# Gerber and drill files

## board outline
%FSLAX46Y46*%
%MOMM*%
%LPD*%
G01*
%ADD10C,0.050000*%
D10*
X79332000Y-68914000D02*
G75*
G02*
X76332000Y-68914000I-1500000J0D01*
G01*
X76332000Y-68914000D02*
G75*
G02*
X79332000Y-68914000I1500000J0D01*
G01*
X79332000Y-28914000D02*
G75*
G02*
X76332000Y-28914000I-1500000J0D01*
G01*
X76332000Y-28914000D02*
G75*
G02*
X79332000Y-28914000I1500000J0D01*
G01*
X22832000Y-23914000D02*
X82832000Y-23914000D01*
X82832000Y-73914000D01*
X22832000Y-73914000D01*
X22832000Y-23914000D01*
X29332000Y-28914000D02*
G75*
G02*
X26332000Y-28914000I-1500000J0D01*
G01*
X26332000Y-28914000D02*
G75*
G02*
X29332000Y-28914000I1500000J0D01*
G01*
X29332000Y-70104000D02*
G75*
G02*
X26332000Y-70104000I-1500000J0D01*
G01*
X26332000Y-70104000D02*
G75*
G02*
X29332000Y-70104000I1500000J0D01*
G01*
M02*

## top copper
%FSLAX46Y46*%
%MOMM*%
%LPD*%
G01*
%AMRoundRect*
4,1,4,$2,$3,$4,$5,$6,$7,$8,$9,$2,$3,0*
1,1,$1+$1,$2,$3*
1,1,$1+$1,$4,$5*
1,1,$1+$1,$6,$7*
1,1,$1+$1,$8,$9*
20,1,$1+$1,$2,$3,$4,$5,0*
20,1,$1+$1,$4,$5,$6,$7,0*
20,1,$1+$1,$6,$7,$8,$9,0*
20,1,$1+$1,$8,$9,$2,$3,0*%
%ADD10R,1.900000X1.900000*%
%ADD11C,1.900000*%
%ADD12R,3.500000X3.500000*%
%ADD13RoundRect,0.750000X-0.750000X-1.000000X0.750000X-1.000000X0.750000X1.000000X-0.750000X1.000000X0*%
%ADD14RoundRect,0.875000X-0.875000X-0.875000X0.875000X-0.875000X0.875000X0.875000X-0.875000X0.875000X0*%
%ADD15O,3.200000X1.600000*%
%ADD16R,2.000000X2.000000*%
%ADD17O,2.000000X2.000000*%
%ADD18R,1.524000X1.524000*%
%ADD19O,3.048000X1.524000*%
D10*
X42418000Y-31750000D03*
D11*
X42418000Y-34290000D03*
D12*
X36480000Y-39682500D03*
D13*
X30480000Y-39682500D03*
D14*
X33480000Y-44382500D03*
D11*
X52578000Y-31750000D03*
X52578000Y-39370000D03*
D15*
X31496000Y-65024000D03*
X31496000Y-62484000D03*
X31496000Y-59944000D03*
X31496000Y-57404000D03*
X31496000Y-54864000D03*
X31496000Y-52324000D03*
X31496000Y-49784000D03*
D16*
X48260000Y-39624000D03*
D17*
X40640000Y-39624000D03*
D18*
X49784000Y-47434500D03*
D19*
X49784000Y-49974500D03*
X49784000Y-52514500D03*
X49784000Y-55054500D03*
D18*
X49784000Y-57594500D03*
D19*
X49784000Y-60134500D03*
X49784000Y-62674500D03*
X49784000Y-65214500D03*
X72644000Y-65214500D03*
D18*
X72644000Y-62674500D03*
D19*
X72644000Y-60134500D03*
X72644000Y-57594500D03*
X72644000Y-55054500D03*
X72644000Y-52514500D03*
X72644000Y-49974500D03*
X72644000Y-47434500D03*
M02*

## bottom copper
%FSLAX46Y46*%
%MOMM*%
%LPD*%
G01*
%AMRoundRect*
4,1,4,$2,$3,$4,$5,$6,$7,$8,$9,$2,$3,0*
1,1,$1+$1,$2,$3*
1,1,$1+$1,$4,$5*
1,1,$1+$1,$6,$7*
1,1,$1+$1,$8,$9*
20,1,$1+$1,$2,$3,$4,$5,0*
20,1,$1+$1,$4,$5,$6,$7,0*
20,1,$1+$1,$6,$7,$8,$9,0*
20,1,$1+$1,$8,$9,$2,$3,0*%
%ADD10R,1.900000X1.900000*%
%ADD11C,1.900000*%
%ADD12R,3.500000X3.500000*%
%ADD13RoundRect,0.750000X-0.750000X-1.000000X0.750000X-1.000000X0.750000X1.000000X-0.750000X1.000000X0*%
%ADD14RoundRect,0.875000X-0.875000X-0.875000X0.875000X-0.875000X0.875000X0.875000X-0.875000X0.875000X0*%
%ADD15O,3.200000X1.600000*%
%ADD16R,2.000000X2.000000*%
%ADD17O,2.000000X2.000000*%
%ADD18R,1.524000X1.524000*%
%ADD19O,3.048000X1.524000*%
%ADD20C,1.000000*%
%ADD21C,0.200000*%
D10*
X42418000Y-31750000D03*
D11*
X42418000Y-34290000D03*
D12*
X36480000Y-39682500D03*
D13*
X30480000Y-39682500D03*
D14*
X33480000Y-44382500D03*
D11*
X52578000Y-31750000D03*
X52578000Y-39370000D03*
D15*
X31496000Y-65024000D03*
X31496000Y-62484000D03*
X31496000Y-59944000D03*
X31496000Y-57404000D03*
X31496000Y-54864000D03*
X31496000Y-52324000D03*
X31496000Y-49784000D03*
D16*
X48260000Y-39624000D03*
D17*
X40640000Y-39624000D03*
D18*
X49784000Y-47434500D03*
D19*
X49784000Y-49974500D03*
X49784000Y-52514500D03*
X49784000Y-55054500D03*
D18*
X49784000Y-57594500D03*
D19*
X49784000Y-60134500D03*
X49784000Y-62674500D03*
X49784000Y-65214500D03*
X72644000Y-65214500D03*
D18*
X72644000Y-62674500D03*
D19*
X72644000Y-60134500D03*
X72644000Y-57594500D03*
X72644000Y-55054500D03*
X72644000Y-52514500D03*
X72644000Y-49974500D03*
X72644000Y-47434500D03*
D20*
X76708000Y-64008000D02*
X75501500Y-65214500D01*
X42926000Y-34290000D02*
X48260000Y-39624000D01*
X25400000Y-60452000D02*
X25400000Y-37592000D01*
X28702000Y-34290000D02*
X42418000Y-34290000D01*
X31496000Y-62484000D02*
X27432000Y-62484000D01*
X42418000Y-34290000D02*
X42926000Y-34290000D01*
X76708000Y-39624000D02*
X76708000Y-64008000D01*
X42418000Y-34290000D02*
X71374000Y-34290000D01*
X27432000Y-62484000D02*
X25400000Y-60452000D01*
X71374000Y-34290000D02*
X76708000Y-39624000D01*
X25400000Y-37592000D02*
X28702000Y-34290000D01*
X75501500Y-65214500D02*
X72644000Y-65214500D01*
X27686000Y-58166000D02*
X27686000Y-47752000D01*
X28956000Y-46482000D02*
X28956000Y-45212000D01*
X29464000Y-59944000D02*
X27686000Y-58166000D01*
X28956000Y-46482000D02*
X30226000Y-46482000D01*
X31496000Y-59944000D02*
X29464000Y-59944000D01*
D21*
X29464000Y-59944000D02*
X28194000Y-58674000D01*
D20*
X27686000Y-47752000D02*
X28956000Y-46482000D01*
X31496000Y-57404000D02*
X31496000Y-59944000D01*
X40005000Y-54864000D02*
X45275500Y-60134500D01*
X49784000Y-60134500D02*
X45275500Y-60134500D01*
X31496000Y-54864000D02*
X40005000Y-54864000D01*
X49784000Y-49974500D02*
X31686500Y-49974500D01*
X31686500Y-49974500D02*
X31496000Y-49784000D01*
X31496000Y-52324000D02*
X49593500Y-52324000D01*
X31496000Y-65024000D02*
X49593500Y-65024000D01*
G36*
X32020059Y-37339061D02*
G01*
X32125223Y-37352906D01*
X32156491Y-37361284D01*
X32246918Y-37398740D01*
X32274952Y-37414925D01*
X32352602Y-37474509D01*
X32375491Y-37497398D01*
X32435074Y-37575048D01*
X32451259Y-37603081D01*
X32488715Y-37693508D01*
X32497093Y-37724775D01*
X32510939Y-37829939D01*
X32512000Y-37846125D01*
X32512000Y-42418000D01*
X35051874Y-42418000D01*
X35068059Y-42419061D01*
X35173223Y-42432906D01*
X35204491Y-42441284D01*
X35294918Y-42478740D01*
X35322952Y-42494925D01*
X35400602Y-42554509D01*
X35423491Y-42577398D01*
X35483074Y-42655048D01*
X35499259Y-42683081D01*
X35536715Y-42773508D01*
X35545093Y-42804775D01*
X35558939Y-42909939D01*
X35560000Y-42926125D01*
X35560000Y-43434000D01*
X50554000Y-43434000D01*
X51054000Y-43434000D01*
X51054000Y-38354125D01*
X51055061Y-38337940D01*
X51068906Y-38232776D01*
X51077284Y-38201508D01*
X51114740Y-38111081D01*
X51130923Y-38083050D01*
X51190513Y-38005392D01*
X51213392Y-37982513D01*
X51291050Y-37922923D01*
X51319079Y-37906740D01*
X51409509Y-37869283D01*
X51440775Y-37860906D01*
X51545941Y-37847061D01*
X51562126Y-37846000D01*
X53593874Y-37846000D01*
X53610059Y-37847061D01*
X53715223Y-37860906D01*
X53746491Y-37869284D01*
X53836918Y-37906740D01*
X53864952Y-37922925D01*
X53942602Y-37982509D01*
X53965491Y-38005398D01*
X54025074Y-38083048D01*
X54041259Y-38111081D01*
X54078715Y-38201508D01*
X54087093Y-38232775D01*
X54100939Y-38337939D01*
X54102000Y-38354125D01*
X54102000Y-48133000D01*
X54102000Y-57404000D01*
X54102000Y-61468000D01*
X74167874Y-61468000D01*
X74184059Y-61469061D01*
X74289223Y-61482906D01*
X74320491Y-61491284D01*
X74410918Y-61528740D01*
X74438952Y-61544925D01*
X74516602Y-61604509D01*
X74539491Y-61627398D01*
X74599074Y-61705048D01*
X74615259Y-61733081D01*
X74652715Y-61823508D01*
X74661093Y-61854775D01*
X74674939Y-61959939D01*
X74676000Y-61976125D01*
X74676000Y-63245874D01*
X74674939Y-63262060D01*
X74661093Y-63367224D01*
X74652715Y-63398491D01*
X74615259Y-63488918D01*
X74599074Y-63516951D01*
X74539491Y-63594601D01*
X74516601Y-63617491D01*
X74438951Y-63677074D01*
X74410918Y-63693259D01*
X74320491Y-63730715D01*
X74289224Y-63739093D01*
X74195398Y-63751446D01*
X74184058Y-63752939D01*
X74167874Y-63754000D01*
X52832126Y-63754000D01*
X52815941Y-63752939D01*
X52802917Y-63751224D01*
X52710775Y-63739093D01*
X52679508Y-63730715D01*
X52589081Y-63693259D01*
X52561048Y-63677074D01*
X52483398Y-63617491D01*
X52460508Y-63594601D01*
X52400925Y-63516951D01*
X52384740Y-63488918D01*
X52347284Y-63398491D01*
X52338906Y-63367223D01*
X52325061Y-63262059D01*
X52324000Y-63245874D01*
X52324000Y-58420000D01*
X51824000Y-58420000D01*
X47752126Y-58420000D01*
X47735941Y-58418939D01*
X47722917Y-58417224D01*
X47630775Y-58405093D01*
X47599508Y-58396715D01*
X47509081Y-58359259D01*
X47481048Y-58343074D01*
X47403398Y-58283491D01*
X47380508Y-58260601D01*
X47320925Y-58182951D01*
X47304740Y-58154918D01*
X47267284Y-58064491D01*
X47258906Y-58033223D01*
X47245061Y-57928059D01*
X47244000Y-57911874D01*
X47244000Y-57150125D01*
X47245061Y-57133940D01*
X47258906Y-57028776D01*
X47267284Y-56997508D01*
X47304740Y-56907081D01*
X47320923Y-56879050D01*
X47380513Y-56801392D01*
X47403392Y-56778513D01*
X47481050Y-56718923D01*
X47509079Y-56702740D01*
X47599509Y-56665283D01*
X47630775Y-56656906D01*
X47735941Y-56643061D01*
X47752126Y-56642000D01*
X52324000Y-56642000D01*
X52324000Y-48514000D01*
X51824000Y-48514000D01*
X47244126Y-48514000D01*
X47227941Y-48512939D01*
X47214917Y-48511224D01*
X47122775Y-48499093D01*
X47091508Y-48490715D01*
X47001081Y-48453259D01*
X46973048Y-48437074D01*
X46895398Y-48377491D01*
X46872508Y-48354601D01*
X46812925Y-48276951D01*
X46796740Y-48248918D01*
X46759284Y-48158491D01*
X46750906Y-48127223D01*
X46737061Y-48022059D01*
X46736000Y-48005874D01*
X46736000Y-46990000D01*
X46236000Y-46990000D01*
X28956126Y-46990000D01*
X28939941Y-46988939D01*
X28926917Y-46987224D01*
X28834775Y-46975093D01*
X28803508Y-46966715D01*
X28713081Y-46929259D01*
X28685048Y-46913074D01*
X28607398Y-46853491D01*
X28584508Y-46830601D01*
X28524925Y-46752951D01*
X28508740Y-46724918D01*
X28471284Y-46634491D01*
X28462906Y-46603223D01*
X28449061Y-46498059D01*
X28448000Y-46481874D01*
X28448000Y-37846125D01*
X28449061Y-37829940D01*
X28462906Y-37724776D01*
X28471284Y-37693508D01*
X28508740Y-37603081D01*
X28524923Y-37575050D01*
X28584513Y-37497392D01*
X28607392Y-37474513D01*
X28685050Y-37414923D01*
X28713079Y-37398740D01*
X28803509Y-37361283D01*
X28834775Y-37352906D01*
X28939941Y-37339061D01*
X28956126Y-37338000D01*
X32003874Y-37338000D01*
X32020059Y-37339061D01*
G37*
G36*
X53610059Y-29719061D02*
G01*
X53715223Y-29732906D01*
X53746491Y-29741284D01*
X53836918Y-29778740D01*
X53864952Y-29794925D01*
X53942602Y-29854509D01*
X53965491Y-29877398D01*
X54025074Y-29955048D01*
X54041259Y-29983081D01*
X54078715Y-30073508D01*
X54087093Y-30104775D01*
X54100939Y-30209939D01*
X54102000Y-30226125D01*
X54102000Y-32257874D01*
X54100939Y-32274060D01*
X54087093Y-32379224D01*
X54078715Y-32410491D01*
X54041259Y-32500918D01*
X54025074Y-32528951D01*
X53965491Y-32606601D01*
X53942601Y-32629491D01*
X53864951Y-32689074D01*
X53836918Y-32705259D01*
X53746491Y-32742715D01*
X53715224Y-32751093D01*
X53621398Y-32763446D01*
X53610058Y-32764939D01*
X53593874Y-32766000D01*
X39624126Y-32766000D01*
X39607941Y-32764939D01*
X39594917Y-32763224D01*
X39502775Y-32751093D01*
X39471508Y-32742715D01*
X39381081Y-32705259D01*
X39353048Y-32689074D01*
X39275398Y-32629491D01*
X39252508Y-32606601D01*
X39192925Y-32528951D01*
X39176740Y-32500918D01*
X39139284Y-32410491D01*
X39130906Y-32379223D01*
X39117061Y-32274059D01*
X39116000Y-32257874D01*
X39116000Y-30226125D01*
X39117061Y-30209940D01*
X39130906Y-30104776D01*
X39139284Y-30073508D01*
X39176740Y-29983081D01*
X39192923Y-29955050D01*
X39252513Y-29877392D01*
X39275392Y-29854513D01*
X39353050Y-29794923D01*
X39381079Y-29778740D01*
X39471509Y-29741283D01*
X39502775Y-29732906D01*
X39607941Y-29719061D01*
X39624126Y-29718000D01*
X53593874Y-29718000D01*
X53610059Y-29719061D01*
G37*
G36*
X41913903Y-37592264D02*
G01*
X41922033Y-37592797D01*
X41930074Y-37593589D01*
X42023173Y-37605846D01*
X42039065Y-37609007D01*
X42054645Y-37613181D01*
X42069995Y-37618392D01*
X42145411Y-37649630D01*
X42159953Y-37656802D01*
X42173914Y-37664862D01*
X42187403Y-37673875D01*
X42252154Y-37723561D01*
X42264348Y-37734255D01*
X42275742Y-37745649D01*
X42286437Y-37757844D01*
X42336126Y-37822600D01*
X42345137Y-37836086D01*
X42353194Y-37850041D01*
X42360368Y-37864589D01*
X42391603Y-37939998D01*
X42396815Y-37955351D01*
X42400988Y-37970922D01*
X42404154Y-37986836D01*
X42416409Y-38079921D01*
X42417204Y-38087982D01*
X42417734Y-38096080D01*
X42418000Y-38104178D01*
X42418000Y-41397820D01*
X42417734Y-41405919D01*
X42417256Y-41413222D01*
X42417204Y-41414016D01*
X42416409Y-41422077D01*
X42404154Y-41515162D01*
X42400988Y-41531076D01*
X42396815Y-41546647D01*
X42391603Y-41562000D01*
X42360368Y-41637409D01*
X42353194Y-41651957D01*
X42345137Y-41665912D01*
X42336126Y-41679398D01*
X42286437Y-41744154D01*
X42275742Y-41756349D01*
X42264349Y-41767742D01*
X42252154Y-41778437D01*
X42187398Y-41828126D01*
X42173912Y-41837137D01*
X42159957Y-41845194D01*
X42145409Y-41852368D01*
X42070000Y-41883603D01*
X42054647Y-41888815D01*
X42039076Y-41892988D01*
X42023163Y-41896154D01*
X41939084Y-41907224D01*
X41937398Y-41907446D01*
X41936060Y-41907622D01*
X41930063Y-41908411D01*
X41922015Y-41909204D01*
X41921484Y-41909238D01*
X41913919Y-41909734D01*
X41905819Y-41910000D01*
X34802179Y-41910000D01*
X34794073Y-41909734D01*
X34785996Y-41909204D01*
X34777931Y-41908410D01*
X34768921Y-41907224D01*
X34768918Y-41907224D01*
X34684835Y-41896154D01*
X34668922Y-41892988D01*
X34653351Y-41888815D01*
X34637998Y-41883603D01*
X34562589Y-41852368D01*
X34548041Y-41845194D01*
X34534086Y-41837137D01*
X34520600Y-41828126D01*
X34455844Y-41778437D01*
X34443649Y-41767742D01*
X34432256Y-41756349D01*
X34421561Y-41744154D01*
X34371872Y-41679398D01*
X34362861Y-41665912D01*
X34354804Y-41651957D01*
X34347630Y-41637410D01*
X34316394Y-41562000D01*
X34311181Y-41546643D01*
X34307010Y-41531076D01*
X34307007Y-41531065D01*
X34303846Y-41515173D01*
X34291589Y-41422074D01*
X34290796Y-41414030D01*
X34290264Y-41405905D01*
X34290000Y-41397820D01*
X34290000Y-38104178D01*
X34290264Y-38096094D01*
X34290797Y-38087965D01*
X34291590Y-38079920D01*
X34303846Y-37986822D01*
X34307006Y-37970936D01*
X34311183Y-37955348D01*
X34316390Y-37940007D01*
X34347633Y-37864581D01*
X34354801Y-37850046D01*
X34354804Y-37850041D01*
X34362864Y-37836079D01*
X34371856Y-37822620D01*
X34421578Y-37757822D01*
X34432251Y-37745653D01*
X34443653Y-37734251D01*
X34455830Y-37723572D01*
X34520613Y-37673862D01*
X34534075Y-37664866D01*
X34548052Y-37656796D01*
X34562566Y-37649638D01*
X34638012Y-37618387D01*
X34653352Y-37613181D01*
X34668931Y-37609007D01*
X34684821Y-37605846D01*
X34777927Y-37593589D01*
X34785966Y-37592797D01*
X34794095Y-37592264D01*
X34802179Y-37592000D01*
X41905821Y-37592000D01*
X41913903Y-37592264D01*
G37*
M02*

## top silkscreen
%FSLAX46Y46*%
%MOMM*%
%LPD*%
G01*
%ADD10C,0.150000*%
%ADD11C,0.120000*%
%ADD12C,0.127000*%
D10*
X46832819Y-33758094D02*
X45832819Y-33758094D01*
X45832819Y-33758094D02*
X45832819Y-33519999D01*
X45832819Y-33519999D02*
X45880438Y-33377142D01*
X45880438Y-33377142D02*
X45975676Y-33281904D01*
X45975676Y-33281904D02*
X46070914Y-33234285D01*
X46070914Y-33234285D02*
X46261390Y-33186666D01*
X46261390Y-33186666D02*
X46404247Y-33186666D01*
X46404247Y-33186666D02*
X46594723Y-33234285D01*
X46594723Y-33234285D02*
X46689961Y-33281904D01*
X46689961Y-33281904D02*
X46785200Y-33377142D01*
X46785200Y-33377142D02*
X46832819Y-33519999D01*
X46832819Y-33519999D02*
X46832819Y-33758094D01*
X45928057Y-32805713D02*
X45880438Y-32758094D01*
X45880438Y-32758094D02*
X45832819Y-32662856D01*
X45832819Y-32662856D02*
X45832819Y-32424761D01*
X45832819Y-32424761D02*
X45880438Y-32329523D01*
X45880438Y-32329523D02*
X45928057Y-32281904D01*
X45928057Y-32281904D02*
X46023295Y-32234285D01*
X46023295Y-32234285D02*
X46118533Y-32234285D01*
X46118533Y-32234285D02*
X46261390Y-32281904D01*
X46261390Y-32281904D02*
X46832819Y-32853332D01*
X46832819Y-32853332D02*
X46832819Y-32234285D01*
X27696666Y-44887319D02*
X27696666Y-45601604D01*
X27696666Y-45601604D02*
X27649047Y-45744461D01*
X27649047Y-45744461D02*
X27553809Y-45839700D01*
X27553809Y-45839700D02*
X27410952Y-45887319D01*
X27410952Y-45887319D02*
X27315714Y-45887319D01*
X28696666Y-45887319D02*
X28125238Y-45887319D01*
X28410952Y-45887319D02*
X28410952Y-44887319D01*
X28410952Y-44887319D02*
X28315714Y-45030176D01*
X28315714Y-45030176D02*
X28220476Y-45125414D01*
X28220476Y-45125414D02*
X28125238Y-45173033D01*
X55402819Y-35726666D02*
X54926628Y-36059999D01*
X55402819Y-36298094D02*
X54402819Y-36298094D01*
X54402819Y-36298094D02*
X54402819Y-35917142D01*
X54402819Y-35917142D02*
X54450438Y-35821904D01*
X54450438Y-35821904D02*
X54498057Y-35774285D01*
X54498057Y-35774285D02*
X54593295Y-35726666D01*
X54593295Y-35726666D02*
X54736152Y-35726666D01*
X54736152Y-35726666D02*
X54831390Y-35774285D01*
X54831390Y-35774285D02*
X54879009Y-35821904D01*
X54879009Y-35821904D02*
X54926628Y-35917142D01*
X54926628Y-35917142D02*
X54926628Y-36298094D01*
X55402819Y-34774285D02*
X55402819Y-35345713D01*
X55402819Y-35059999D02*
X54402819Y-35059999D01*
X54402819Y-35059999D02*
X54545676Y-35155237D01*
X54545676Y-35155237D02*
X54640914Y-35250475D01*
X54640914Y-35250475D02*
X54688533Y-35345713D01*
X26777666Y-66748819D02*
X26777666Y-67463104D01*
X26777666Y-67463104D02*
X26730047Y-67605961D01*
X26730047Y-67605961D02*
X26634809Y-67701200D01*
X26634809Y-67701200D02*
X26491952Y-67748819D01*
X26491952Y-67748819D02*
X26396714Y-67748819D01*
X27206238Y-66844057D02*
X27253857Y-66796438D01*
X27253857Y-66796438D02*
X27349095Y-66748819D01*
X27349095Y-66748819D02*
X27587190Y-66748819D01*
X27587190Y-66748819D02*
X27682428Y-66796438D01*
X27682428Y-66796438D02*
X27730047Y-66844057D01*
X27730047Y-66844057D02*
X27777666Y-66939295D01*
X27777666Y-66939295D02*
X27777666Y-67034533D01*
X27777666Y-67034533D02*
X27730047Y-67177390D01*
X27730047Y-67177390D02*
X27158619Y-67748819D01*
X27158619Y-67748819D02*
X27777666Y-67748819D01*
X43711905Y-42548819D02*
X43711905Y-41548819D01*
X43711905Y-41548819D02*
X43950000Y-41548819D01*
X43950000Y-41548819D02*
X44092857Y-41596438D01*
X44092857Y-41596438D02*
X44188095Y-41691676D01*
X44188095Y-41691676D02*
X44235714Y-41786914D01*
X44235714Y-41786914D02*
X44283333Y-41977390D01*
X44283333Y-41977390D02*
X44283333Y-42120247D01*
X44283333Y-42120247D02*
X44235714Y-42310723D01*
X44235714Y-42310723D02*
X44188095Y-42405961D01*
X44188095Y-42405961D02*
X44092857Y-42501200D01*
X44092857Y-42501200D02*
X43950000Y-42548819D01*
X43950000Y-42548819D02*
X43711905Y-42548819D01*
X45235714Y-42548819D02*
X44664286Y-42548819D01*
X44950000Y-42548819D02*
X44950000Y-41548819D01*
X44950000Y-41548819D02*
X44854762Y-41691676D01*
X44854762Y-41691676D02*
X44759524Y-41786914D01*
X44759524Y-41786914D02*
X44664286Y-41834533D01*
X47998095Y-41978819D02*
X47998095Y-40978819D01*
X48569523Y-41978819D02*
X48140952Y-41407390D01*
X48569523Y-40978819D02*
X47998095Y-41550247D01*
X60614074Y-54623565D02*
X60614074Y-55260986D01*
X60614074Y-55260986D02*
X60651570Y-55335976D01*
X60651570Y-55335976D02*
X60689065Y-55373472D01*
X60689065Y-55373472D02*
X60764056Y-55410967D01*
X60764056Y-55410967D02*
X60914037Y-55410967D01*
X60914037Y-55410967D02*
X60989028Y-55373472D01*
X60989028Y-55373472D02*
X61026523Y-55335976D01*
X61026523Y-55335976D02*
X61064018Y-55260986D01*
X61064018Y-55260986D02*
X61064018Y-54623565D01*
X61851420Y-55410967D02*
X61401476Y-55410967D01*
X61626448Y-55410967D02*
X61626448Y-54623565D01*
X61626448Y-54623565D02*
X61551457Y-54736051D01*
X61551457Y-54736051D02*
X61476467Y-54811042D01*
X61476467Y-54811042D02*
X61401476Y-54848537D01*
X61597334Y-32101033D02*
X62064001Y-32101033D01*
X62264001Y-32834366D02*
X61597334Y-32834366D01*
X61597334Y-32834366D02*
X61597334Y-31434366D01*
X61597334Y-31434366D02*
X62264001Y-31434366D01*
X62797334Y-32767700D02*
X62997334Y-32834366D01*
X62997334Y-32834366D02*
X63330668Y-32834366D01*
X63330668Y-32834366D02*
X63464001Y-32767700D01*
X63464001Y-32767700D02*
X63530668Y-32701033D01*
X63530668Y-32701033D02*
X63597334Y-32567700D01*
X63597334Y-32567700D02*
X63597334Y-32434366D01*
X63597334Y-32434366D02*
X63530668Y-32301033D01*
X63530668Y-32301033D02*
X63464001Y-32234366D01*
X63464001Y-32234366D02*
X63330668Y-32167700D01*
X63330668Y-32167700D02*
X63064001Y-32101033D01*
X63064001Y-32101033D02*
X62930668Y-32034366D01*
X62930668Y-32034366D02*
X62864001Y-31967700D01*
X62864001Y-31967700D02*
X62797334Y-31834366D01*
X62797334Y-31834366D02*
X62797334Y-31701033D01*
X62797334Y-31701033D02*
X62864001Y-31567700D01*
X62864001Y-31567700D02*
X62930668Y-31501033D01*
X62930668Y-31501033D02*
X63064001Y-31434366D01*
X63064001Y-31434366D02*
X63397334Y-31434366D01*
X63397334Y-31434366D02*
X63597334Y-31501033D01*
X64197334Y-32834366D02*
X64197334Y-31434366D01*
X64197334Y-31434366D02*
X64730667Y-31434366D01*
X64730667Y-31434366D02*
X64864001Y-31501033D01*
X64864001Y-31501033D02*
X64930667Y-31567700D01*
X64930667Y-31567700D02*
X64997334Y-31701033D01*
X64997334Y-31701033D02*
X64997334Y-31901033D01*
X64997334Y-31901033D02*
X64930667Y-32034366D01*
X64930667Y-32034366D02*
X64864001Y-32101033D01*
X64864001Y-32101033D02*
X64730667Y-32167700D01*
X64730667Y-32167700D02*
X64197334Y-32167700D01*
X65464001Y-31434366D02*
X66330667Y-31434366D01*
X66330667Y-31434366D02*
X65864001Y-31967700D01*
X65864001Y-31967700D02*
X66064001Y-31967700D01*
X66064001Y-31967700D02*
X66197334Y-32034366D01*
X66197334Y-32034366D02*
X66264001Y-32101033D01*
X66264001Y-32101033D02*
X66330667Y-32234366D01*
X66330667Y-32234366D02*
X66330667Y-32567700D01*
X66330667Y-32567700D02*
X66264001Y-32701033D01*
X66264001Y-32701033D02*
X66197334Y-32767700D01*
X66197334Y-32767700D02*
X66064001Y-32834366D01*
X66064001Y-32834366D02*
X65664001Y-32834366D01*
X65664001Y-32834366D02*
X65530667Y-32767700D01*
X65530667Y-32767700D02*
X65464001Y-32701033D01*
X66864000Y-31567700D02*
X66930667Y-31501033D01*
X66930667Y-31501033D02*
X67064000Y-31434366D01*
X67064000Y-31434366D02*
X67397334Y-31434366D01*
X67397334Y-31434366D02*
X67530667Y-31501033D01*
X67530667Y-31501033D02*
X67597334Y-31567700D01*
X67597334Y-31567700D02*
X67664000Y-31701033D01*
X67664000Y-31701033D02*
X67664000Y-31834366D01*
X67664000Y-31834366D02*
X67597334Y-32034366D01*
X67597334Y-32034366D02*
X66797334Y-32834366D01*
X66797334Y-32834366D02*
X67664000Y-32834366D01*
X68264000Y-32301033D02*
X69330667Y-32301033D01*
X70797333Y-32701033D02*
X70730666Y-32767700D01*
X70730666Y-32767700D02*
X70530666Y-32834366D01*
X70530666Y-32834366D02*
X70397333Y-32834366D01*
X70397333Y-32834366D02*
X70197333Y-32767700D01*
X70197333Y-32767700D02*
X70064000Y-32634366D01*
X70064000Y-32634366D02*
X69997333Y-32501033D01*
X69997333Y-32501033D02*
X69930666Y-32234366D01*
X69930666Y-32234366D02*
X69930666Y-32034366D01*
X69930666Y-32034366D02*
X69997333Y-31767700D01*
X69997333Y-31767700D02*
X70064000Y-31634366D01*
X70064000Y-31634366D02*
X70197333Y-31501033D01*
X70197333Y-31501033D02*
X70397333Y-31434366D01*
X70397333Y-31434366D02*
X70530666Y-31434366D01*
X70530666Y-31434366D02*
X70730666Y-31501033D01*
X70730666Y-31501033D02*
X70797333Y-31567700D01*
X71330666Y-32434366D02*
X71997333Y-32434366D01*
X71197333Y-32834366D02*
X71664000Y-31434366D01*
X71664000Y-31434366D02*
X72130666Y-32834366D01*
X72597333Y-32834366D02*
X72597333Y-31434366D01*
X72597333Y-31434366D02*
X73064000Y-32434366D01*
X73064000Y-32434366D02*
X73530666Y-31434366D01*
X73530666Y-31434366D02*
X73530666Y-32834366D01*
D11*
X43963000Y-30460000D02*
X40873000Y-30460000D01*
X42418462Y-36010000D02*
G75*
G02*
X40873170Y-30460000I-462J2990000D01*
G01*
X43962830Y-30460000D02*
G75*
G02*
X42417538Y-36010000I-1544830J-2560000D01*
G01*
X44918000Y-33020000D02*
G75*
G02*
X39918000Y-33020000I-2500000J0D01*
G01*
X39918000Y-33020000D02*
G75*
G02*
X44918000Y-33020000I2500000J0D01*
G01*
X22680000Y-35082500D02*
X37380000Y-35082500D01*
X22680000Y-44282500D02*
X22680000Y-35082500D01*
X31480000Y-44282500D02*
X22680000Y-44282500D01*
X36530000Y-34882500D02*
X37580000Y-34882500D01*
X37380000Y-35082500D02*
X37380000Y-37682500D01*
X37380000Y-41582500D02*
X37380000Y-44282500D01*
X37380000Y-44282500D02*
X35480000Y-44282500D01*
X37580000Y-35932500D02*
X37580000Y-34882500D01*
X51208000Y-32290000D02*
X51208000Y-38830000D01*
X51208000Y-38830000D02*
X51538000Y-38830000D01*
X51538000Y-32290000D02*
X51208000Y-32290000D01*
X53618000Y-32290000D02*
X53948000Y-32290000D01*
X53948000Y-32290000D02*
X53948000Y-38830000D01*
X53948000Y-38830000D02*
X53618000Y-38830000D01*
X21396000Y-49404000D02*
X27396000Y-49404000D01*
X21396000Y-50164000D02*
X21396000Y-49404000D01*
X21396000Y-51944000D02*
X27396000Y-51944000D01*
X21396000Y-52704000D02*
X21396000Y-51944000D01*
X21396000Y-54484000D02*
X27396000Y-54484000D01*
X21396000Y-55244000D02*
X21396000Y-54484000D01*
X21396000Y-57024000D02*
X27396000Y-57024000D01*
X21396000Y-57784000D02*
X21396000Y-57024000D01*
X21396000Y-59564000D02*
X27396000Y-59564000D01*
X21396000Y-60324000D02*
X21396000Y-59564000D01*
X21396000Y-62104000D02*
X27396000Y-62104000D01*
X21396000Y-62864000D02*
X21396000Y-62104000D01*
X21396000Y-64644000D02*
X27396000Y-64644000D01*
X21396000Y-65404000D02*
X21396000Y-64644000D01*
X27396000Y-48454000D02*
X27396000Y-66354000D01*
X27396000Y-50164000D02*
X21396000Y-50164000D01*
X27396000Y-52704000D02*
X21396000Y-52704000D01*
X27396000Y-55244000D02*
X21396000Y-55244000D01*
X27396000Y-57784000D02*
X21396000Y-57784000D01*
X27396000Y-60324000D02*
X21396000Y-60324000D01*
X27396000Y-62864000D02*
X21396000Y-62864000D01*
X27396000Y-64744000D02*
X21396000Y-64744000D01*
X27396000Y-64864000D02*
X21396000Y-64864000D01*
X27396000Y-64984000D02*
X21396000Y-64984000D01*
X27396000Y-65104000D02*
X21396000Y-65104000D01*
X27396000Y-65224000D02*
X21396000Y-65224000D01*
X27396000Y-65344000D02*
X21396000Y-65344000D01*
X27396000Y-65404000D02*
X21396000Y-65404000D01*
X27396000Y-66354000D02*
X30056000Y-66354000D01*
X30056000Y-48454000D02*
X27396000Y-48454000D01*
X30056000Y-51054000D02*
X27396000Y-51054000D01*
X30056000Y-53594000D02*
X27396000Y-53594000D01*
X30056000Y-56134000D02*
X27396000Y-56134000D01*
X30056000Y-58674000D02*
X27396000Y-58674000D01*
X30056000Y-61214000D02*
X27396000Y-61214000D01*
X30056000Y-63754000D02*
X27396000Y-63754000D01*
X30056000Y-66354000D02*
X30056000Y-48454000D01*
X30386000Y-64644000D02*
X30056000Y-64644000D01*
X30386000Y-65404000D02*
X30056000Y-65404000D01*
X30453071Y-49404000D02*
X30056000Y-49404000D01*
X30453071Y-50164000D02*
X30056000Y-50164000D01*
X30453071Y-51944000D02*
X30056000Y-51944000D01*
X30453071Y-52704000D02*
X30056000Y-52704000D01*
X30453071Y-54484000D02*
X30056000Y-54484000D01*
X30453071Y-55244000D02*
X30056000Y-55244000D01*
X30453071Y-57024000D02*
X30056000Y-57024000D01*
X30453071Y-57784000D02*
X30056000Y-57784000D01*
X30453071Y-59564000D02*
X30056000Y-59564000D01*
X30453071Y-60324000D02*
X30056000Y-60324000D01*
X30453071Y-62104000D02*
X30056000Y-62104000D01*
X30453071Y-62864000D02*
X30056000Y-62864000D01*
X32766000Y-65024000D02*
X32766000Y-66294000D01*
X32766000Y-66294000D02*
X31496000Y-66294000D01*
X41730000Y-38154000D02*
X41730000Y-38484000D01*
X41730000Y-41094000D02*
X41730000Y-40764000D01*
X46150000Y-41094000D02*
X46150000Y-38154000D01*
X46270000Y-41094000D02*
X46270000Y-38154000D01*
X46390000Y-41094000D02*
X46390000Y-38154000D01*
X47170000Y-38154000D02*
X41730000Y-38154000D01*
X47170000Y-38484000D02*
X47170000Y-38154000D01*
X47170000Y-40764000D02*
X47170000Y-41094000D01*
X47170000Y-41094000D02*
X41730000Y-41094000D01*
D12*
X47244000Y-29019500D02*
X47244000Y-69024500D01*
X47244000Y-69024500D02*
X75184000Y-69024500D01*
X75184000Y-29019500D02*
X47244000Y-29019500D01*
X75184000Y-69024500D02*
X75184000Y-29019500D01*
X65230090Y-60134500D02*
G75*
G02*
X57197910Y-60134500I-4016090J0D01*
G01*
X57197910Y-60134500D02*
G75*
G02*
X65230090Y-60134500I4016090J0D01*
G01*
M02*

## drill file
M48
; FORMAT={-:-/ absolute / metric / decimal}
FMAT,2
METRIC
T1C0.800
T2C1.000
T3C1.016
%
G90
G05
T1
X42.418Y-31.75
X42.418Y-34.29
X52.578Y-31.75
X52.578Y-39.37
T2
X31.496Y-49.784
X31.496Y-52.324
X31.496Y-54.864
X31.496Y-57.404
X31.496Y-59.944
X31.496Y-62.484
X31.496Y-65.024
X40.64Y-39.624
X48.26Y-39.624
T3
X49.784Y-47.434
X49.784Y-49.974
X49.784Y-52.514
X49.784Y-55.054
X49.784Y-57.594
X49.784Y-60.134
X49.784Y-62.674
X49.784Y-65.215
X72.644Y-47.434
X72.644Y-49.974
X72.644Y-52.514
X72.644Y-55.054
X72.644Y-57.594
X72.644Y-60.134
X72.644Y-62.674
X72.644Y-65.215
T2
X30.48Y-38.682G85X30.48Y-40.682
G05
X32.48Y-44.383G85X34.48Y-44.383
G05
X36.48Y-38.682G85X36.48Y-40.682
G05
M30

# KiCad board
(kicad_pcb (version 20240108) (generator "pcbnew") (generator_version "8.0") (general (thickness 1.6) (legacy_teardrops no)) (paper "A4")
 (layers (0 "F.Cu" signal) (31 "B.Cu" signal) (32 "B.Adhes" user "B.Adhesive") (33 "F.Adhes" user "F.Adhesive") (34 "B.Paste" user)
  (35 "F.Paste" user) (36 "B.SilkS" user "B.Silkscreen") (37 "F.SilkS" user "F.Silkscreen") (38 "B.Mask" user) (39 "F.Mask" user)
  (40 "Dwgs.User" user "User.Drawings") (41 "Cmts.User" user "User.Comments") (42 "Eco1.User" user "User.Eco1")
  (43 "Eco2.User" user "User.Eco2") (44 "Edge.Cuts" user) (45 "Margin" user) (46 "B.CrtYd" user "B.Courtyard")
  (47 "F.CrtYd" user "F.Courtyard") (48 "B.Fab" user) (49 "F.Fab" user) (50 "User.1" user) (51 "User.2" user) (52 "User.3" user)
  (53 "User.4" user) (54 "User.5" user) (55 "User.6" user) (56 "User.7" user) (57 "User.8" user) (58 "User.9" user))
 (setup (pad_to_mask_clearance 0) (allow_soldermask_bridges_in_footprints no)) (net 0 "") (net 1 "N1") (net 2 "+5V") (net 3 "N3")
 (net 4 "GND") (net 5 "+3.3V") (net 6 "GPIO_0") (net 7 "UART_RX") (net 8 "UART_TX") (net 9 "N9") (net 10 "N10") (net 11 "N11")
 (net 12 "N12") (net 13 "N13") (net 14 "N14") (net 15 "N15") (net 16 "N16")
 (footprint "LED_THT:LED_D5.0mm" (layer "F.Cu") (at 42.418 31.75 -90)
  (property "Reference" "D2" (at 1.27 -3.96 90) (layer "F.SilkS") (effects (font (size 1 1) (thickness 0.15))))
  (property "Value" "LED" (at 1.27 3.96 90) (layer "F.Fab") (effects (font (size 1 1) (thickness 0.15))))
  (fp_line (start -1.29 -1.545) (end -1.29 1.545) (stroke (width 0.12) (type solid)) (layer "F.SilkS"))
  (fp_arc (start 4.26 -0.000462) (mid 2.072002 2.880433) (end -1.29 1.54483) (stroke (width 0.12) (type solid)) (layer "F.SilkS"))
  (fp_arc (start -1.29 -1.54483) (mid 2.072002 -2.880433) (end 4.26 0.000462) (stroke (width 0.12) (type solid)) (layer "F.SilkS"))
  (fp_circle (center 1.27 0) (end 3.77 0) (stroke (width 0.12) (type solid)) (fill none) (layer "F.SilkS"))
  (pad "1" thru_hole rect (at 0 0 270) (size 1.9 1.9) (drill 0.8) (layers "*.Cu" "*.Mask") (remove_unused_layers no) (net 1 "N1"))
  (pad "2" thru_hole circle (at 2.54 0 270) (size 1.9 1.9) (drill 0.8) (layers "*.Cu" "*.Mask") (remove_unused_layers no) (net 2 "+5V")))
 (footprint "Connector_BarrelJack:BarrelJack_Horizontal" (layer "F.Cu") (at 36.48 39.6825)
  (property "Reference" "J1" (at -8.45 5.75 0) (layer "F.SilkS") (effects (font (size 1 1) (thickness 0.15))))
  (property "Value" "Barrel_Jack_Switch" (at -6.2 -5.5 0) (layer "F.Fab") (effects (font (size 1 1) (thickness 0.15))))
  (fp_line (start -13.8 -4.6) (end 0.9 -4.6) (stroke (width 0.12) (type solid)) (layer "F.SilkS"))
  (fp_line (start -13.8 4.6) (end -13.8 -4.6) (stroke (width 0.12) (type solid)) (layer "F.SilkS"))
  (fp_line (start -5 4.6) (end -13.8 4.6) (stroke (width 0.12) (type solid)) (layer "F.SilkS"))
  (fp_line (start 0.05 -4.8) (end 1.1 -4.8) (stroke (width 0.12) (type solid)) (layer "F.SilkS"))
  (fp_line (start 0.9 -4.6) (end 0.9 -2) (stroke (width 0.12) (type solid)) (layer "F.SilkS"))
  (fp_line (start 0.9 1.9) (end 0.9 4.6) (stroke (width 0.12) (type solid)) (layer "F.SilkS"))
  (fp_line (start 0.9 4.6) (end -1 4.6) (stroke (width 0.12) (type solid)) (layer "F.SilkS"))
  (fp_line (start 1.1 -3.75) (end 1.1 -4.8) (stroke (width 0.12) (type solid)) (layer "F.SilkS"))
  (pad "1" thru_hole rect (at 0 0) (size 3.5 3.5) (drill oval 1 3) (layers "*.Cu" "*.Mask") (remove_unused_layers no) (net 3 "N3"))
  (pad "2" thru_hole roundrect (at -6 0) (size 3 3.5) (drill oval 1 3) (layers "*.Cu" "*.Mask") (remove_unused_layers no)
   (roundrect_rratio 0.25) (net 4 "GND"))
  (pad "3" thru_hole roundrect (at -3 4.7) (size 3.5 3.5) (drill oval 3 1) (layers "*.Cu" "*.Mask") (remove_unused_layers no)
   (roundrect_rratio 0.25) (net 4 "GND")))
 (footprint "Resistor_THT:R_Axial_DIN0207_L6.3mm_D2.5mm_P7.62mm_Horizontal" (layer "F.Cu") (at 52.578 31.75 -90)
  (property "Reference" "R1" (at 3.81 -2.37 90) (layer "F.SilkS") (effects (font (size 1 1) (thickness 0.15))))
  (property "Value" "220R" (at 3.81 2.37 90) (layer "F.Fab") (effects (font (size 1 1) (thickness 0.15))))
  (fp_line (start 0.54 1.37) (end 7.08 1.37) (stroke (width 0.12) (type solid)) (layer "F.SilkS"))
  (fp_line (start 7.08 1.37) (end 7.08 1.04) (stroke (width 0.12) (type solid)) (layer "F.SilkS"))
  (fp_line (start 0.54 1.04) (end 0.54 1.37) (stroke (width 0.12) (type solid)) (layer "F.SilkS"))
  (fp_line (start 0.54 -1.04) (end 0.54 -1.37) (stroke (width 0.12) (type solid)) (layer "F.SilkS"))
  (fp_line (start 0.54 -1.37) (end 7.08 -1.37) (stroke (width 0.12) (type solid)) (layer "F.SilkS"))
  (fp_line (start 7.08 -1.37) (end 7.08 -1.04) (stroke (width 0.12) (type solid)) (layer "F.SilkS"))
  (pad "1" thru_hole circle (at 0 0 270) (size 1.9 1.9) (drill 0.8) (layers "*.Cu" "*.Mask") (remove_unused_layers no) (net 1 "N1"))
  (pad "2" thru_hole circle (at 7.62 0 270) (size 1.9 1.9) (drill 0.8) (layers "*.Cu" "*.Mask") (remove_unused_layers no) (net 4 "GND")))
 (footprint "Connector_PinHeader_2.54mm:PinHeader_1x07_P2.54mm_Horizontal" (layer "F.Cu") (at 31.496 65.024 180)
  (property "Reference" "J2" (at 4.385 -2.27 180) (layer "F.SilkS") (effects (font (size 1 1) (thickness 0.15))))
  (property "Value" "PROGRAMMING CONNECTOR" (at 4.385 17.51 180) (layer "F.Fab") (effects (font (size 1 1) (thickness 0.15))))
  (fp_line (start 10.1 15.62) (end 4.1 15.62) (stroke (width 0.12) (type solid)) (layer "F.SilkS"))
  (fp_line (start 10.1 14.86) (end 10.1 15.62) (stroke (width 0.12) (type solid)) (layer "F.SilkS"))
  (fp_line (start 10.1 13.08) (end 4.1 13.08) (stroke (width 0.12) (type solid)) (layer "F.SilkS"))
  (fp_line (start 10.1 12.32) (end 10.1 13.08) (stroke (width 0.12) (type solid)) (layer "F.SilkS"))
  (fp_line (start 10.1 10.54) (end 4.1 10.54) (stroke (width 0.12) (type solid)) (layer "F.SilkS"))
  (fp_line (start 10.1 9.78) (end 10.1 10.54) (stroke (width 0.12) (type solid)) (layer "F.SilkS"))
  (fp_line (start 10.1 8) (end 4.1 8) (stroke (width 0.12) (type solid)) (layer "F.SilkS"))
  (fp_line (start 10.1 7.24) (end 10.1 8) (stroke (width 0.12) (type solid)) (layer "F.SilkS"))
  (fp_line (start 10.1 5.46) (end 4.1 5.46) (stroke (width 0.12) (type solid)) (layer "F.SilkS"))
  (fp_line (start 10.1 4.7) (end 10.1 5.46) (stroke (width 0.12) (type solid)) (layer "F.SilkS"))
  (fp_line (start 10.1 2.92) (end 4.1 2.92) (stroke (width 0.12) (type solid)) (layer "F.SilkS"))
  (fp_line (start 10.1 2.16) (end 10.1 2.92) (stroke (width 0.12) (type solid)) (layer "F.SilkS"))
  (fp_line (start 10.1 0.38) (end 4.1 0.38) (stroke (width 0.12) (type solid)) (layer "F.SilkS"))
  (fp_line (start 10.1 -0.38) (end 10.1 0.38) (stroke (width 0.12) (type solid)) (layer "F.SilkS"))
  (fp_line (start 4.1 16.57) (end 4.1 -1.33) (stroke (width 0.12) (type solid)) (layer "F.SilkS"))
  (fp_line (start 4.1 14.86) (end 10.1 14.86) (stroke (width 0.12) (type solid)) (layer "F.SilkS"))
  (fp_line (start 4.1 12.32) (end 10.1 12.32) (stroke (width 0.12) (type solid)) (layer "F.SilkS"))
  (fp_line (start 4.1 9.78) (end 10.1 9.78) (stroke (width 0.12) (type solid)) (layer "F.SilkS"))
  (fp_line (start 4.1 7.24) (end 10.1 7.24) (stroke (width 0.12) (type solid)) (layer "F.SilkS"))
  (fp_line (start 4.1 4.7) (end 10.1 4.7) (stroke (width 0.12) (type solid)) (layer "F.SilkS"))
  (fp_line (start 4.1 2.16) (end 10.1 2.16) (stroke (width 0.12) (type solid)) (layer "F.SilkS"))
  (fp_line (start 4.1 0.28) (end 10.1 0.28) (stroke (width 0.12) (type solid)) (layer "F.SilkS"))
  (fp_line (start 4.1 0.16) (end 10.1 0.16) (stroke (width 0.12) (type solid)) (layer "F.SilkS"))
  (fp_line (start 4.1 0.04) (end 10.1 0.04) (stroke (width 0.12) (type solid)) (layer "F.SilkS"))
  (fp_line (start 4.1 -0.08) (end 10.1 -0.08) (stroke (width 0.12) (type solid)) (layer "F.SilkS"))
  (fp_line (start 4.1 -0.2) (end 10.1 -0.2) (stroke (width 0.12) (type solid)) (layer "F.SilkS"))
  (fp_line (start 4.1 -0.32) (end 10.1 -0.32) (stroke (width 0.12) (type solid)) (layer "F.SilkS"))
  (fp_line (start 4.1 -0.38) (end 10.1 -0.38) (stroke (width 0.12) (type solid)) (layer "F.SilkS"))
  (fp_line (start 4.1 -1.33) (end 1.44 -1.33) (stroke (width 0.12) (type solid)) (layer "F.SilkS"))
  (fp_line (start 1.44 16.57) (end 4.1 16.57) (stroke (width 0.12) (type solid)) (layer "F.SilkS"))
  (fp_line (start 1.44 13.97) (end 4.1 13.97) (stroke (width 0.12) (type solid)) (layer "F.SilkS"))
  (fp_line (start 1.44 11.43) (end 4.1 11.43) (stroke (width 0.12) (type solid)) (layer "F.SilkS"))
  (fp_line (start 1.44 8.89) (end 4.1 8.89) (stroke (width 0.12) (type solid)) (layer "F.SilkS"))
  (fp_line (start 1.44 6.35) (end 4.1 6.35) (stroke (width 0.12) (type solid)) (layer "F.SilkS"))
  (fp_line (start 1.44 3.81) (end 4.1 3.81) (stroke (width 0.12) (type solid)) (layer "F.SilkS"))
  (fp_line (start 1.44 1.27) (end 4.1 1.27) (stroke (width 0.12) (type solid)) (layer "F.SilkS"))
  (fp_line (start 1.44 -1.33) (end 1.44 16.57) (stroke (width 0.12) (type solid)) (layer "F.SilkS"))
  (fp_line (start 1.11 0.38) (end 1.44 0.38) (stroke (width 0.12) (type solid)) (layer "F.SilkS"))
  (fp_line (start 1.11 -0.38) (end 1.44 -0.38) (stroke (width 0.12) (type solid)) (layer "F.SilkS"))
  (fp_line (start 1.042929 15.62) (end 1.44 15.62) (stroke (width 0.12) (type solid)) (layer "F.SilkS"))
  (fp_line (start 1.042929 14.86) (end 1.44 14.86) (stroke (width 0.12) (type solid)) (layer "F.SilkS"))
  (fp_line (start 1.042929 13.08) (end 1.44 13.08) (stroke (width 0.12) (type solid)) (layer "F.SilkS"))
  (fp_line (start 1.042929 12.32) (end 1.44 12.32) (stroke (width 0.12) (type solid)) (layer "F.SilkS"))
  (fp_line (start 1.042929 10.54) (end 1.44 10.54) (stroke (width 0.12) (type solid)) (layer "F.SilkS"))
  (fp_line (start 1.042929 9.78) (end 1.44 9.78) (stroke (width 0.12) (type solid)) (layer "F.SilkS"))
  (fp_line (start 1.042929 8) (end 1.44 8) (stroke (width 0.12) (type solid)) (layer "F.SilkS"))
  (fp_line (start 1.042929 7.24) (end 1.44 7.24) (stroke (width 0.12) (type solid)) (layer "F.SilkS"))
  (fp_line (start 1.042929 5.46) (end 1.44 5.46) (stroke (width 0.12) (type solid)) (layer "F.SilkS"))
  (fp_line (start 1.042929 4.7) (end 1.44 4.7) (stroke (width 0.12) (type solid)) (layer "F.SilkS"))
  (fp_line (start 1.042929 2.92) (end 1.44 2.92) (stroke (width 0.12) (type solid)) (layer "F.SilkS"))
  (fp_line (start 1.042929 2.16) (end 1.44 2.16) (stroke (width 0.12) (type solid)) (layer "F.SilkS"))
  (fp_line (start -1.27 0) (end -1.27 -1.27) (stroke (width 0.12) (type solid)) (layer "F.SilkS"))
  (fp_line (start -1.27 -1.27) (end 0 -1.27) (stroke (width 0.12) (type solid)) (layer "F.SilkS"))
  (pad "1" thru_hole oval (at 0 0 180) (size 3.2 1.6) (drill 1) (layers "*.Cu" "*.Mask") (remove_unused_layers no) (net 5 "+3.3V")
   (solder_mask_margin 0.102))
  (pad "2" thru_hole oval (at 0 2.54 180) (size 3.2 1.6) (drill 1) (layers "*.Cu" "*.Mask") (remove_unused_layers no) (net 2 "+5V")
   (solder_mask_margin 0.102))
  (pad "3" thru_hole oval (at 0 5.08 180) (size 3.2 1.6) (drill 1) (layers "*.Cu" "*.Mask") (remove_unused_layers no) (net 4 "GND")
   (solder_mask_margin 0.102))
  (pad "4" thru_hole oval (at 0 7.62 180) (size 3.2 1.6) (drill 1) (layers "*.Cu" "*.Mask") (remove_unused_layers no) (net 4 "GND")
   (solder_mask_margin 0.102))
  (pad "5" thru_hole oval (at 0 10.16 180) (size 3.2 1.6) (drill 1) (layers "*.Cu" "*.Mask") (remove_unused_layers no) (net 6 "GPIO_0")
   (solder_mask_margin 0.102))
  (pad "6" thru_hole oval (at 0 12.7 180) (size 3.2 1.6) (drill 1) (layers "*.Cu" "*.Mask") (remove_unused_layers no) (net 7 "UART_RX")
   (solder_mask_margin 0.102))
  (pad "7" thru_hole oval (at 0 15.24 180) (size 3.2 1.6) (drill 1) (layers "*.Cu" "*.Mask") (remove_unused_layers no) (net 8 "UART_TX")
   (solder_mask_margin 0.102)))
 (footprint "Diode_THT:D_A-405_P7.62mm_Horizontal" (layer "F.Cu") (at 48.26 39.624 180)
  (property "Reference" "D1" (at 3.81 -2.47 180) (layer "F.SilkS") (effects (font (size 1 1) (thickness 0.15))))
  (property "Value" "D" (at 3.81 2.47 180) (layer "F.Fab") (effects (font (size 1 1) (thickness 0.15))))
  (fp_line (start 6.53 1.47) (end 6.53 1.14) (stroke (width 0.12) (type solid)) (layer "F.SilkS"))
  (fp_line (start 6.53 -1.47) (end 6.53 -1.14) (stroke (width 0.12) (type solid)) (layer "F.SilkS"))
  (fp_line (start 2.11 -1.47) (end 2.11 1.47) (stroke (width 0.12) (type solid)) (layer "F.SilkS"))
  (fp_line (start 1.99 -1.47) (end 1.99 1.47) (stroke (width 0.12) (type solid)) (layer "F.SilkS"))
  (fp_line (start 1.87 -1.47) (end 1.87 1.47) (stroke (width 0.12) (type solid)) (layer "F.SilkS"))
  (fp_line (start 1.09 1.47) (end 6.53 1.47) (stroke (width 0.12) (type solid)) (layer "F.SilkS"))
  (fp_line (start 1.09 1.14) (end 1.09 1.47) (stroke (width 0.12) (type solid)) (layer "F.SilkS"))
  (fp_line (start 1.09 -1.14) (end 1.09 -1.47) (stroke (width 0.12) (type solid)) (layer "F.SilkS"))
  (fp_line (start 1.09 -1.47) (end 6.53 -1.47) (stroke (width 0.12) (type solid)) (layer "F.SilkS"))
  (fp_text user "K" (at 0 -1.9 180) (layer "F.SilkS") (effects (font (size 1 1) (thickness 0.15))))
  (pad "1" thru_hole rect (at 0 0 180) (size 2 2) (drill 1) (layers "*.Cu" "*.Mask") (remove_unused_layers no) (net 2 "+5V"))
  (pad "2" thru_hole oval (at 7.62 0 180) (size 2 2) (drill 1) (layers "*.Cu" "*.Mask") (remove_unused_layers no) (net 3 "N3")))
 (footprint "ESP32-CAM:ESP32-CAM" (layer "F.Cu") (at 61.214 55.0545)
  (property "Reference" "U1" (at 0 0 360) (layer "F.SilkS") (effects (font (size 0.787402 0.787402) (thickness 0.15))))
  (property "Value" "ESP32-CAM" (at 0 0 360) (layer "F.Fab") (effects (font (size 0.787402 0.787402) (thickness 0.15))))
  (fp_line (start -13.97 -26.035) (end -13.97 13.97) (stroke (width 0.127) (type solid)) (layer "F.SilkS"))
  (fp_line (start -13.97 13.97) (end 13.97 13.97) (stroke (width 0.127) (type solid)) (layer "F.SilkS"))
  (fp_line (start 13.97 -26.035) (end -13.97 -26.035) (stroke (width 0.127) (type solid)) (layer "F.SilkS"))
  (fp_line (start 13.97 13.97) (end 13.97 -26.035) (stroke (width 0.127) (type solid)) (layer "F.SilkS"))
  (fp_circle (center 0 5.08) (end 4.01609 5.08) (stroke (width 0.127) (type solid)) (fill none) (layer "F.SilkS"))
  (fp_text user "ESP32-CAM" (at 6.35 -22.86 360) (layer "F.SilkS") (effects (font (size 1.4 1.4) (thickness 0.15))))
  (pad "P$1" thru_hole rect (at -11.43 -7.62) (size 1.524 1.524) (drill 1.016) (layers "*.Cu" "*.Mask") (remove_unused_layers no)
   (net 4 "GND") (solder_mask_margin 0.102))
  (pad "P$2" thru_hole oval (at -11.43 -5.08) (size 3.048 1.524) (drill 1.016) (layers "*.Cu" "*.Mask") (remove_unused_layers no)
   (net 8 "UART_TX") (solder_mask_margin 0.102))
  (pad "P$3" thru_hole oval (at -11.43 -2.54) (size 3.048 1.524) (drill 1.016) (layers "*.Cu" "*.Mask") (remove_unused_layers no)
   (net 7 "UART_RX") (solder_mask_margin 0.102))
  (pad "P$4" thru_hole oval (at -11.43 0) (size 3.048 1.524) (drill 1.016) (layers "*.Cu" "*.Mask") (remove_unused_layers no) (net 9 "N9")
   (solder_mask_margin 0.102))
  (pad "P$5" thru_hole rect (at -11.43 2.54) (size 1.524 1.524) (drill 1.016) (layers "*.Cu" "*.Mask") (remove_unused_layers no)
   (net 4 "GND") (solder_mask_margin 0.102))
  (pad "P$6" thru_hole oval (at -11.43 5.08) (size 3.048 1.524) (drill 1.016) (layers "*.Cu" "*.Mask") (remove_unused_layers no)
   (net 6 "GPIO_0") (solder_mask_margin 0.102))
  (pad "P$7" thru_hole oval (at -11.43 7.62) (size 3.048 1.524) (drill 1.016) (layers "*.Cu" "*.Mask") (remove_unused_layers no)
   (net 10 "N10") (solder_mask_margin 0.102))
  (pad "P$8" thru_hole oval (at -11.43 10.16) (size 3.048 1.524) (drill 1.016) (layers "*.Cu" "*.Mask") (remove_unused_layers no)
   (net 5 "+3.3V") (solder_mask_margin 0.102))
  (pad "P$9" thru_hole oval (at 11.43 10.16) (size 3.048 1.524) (drill 1.016) (layers "*.Cu" "*.Mask") (remove_unused_layers no)
   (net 2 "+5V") (solder_mask_margin 0.102))
  (pad "P$10" thru_hole rect (at 11.43 7.62) (size 1.524 1.524) (drill 1.016) (layers "*.Cu" "*.Mask") (remove_unused_layers no)
   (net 4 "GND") (solder_mask_margin 0.102))
  (pad "P$11" thru_hole oval (at 11.43 5.08) (size 3.048 1.524) (drill 1.016) (layers "*.Cu" "*.Mask") (remove_unused_layers no)
   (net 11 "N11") (solder_mask_margin 0.102))
  (pad "P$12" thru_hole oval (at 11.43 2.54) (size 3.048 1.524) (drill 1.016) (layers "*.Cu" "*.Mask") (remove_unused_layers no)
   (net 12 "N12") (solder_mask_margin 0.102))
  (pad "P$13" thru_hole oval (at 11.43 0) (size 3.048 1.524) (drill 1.016) (layers "*.Cu" "*.Mask") (remove_unused_layers no) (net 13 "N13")
   (solder_mask_margin 0.102))
  (pad "P$14" thru_hole oval (at 11.43 -2.54) (size 3.048 1.524) (drill 1.016) (layers "*.Cu" "*.Mask") (remove_unused_layers no)
   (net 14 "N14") (solder_mask_margin 0.102))
  (pad "P$15" thru_hole oval (at 11.43 -5.08) (size 3.048 1.524) (drill 1.016) (layers "*.Cu" "*.Mask") (remove_unused_layers no)
   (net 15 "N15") (solder_mask_margin 0.102))
  (pad "P$16" thru_hole oval (at 11.43 -7.62) (size 3.048 1.524) (drill 1.016) (layers "*.Cu" "*.Mask") (remove_unused_layers no)
   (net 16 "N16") (solder_mask_margin 0.102)))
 (gr_circle (center 77.832 68.914) (end 79.332 68.914) (stroke (width 0.05) (type default)) (fill none) (layer "Edge.Cuts"))
 (gr_circle (center 77.832 28.914) (end 79.332 28.914) (stroke (width 0.05) (type default)) (fill none) (layer "Edge.Cuts"))
 (gr_rect (start 22.832 23.914) (end 82.832 73.914) (stroke (width 0.05) (type default)) (fill none) (layer "Edge.Cuts"))
 (gr_circle (center 27.832 28.914) (end 29.332 28.914) (stroke (width 0.05) (type default)) (fill none) (layer "Edge.Cuts"))
 (gr_circle (center 27.832 70.104) (end 29.332 70.104) (stroke (width 0.05) (type default)) (fill none) (layer "Edge.Cuts"))
 (segment (start 76.708 64.008) (end 75.5015 65.2145) (width 1) (layer "B.Cu") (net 2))
 (segment (start 42.926 34.29) (end 48.26 39.624) (width 1) (layer "B.Cu") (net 2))
 (segment (start 25.4 60.452) (end 25.4 37.592) (width 1) (layer "B.Cu") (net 2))
 (segment (start 28.702 34.29) (end 42.418 34.29) (width 1) (layer "B.Cu") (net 2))
 (segment (start 31.496 62.484) (end 27.432 62.484) (width 1) (layer "B.Cu") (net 2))
 (segment (start 42.418 34.29) (end 42.926 34.29) (width 1) (layer "B.Cu") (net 2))
 (segment (start 76.708 39.624) (end 76.708 64.008) (width 1) (layer "B.Cu") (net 2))
 (segment (start 42.418 34.29) (end 71.374 34.29) (width 1) (layer "B.Cu") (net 2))
 (segment (start 27.432 62.484) (end 25.4 60.452) (width 1) (layer "B.Cu") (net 2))
 (segment (start 71.374 34.29) (end 76.708 39.624) (width 1) (layer "B.Cu") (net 2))
 (segment (start 25.4 37.592) (end 28.702 34.29) (width 1) (layer "B.Cu") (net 2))
 (segment (start 75.5015 65.2145) (end 72.644 65.2145) (width 1) (layer "B.Cu") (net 2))
 (segment (start 27.686 58.166) (end 27.686 47.752) (width 1) (layer "B.Cu") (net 4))
 (segment (start 28.956 46.482) (end 28.956 45.212) (width 1) (layer "B.Cu") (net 4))
 (segment (start 29.464 59.944) (end 27.686 58.166) (width 1) (layer "B.Cu") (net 4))
 (segment (start 28.956 46.482) (end 30.226 46.482) (width 1) (layer "B.Cu") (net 4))
 (segment (start 31.496 59.944) (end 29.464 59.944) (width 1) (layer "B.Cu") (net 4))
 (segment (start 29.464 59.944) (end 28.194 58.674) (width 0.2) (layer "B.Cu") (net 4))
 (segment (start 27.686 47.752) (end 28.956 46.482) (width 1) (layer "B.Cu") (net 4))
 (segment (start 31.496 57.404) (end 31.496 59.944) (width 1) (layer "B.Cu") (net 4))
 (segment (start 40.005 54.864) (end 45.2755 60.1345) (width 1) (layer "B.Cu") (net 6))
 (segment (start 49.784 60.1345) (end 45.2755 60.1345) (width 1) (layer "B.Cu") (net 6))
 (segment (start 31.496 54.864) (end 40.005 54.864) (width 1) (layer "B.Cu") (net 6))
 (segment (start 49.784 49.9745) (end 31.6865 49.9745) (width 1) (layer "B.Cu") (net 8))
 (segment (start 31.6865 49.9745) (end 31.496 49.784) (width 1) (layer "B.Cu") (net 8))
 (segment (start 31.496 52.324) (end 49.5935 52.324) (width 1) (layer "B.Cu") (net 7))
 (segment (start 31.496 65.024) (end 49.5935 65.024) (width 1) (layer "B.Cu") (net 5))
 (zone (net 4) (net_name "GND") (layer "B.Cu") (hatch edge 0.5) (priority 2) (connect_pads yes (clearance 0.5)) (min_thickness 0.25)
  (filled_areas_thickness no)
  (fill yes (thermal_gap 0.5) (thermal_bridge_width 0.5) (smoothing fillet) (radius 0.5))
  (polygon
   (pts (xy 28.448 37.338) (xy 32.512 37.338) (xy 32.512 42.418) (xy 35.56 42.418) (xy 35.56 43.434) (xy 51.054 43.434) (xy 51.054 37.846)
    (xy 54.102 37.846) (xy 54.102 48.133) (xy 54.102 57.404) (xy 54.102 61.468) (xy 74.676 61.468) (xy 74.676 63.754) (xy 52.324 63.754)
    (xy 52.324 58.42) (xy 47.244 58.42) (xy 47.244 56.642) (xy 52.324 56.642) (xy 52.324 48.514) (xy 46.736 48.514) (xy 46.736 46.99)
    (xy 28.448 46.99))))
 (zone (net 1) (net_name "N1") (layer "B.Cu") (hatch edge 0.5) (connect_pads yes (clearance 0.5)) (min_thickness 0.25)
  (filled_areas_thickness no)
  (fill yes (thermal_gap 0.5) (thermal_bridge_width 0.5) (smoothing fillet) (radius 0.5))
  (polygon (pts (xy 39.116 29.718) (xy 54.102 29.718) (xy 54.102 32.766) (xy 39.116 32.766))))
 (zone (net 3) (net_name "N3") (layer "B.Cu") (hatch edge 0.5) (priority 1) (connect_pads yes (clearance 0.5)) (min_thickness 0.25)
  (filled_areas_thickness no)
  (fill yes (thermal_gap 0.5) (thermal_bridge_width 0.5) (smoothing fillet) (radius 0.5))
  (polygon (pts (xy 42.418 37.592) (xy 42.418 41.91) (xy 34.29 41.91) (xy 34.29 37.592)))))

